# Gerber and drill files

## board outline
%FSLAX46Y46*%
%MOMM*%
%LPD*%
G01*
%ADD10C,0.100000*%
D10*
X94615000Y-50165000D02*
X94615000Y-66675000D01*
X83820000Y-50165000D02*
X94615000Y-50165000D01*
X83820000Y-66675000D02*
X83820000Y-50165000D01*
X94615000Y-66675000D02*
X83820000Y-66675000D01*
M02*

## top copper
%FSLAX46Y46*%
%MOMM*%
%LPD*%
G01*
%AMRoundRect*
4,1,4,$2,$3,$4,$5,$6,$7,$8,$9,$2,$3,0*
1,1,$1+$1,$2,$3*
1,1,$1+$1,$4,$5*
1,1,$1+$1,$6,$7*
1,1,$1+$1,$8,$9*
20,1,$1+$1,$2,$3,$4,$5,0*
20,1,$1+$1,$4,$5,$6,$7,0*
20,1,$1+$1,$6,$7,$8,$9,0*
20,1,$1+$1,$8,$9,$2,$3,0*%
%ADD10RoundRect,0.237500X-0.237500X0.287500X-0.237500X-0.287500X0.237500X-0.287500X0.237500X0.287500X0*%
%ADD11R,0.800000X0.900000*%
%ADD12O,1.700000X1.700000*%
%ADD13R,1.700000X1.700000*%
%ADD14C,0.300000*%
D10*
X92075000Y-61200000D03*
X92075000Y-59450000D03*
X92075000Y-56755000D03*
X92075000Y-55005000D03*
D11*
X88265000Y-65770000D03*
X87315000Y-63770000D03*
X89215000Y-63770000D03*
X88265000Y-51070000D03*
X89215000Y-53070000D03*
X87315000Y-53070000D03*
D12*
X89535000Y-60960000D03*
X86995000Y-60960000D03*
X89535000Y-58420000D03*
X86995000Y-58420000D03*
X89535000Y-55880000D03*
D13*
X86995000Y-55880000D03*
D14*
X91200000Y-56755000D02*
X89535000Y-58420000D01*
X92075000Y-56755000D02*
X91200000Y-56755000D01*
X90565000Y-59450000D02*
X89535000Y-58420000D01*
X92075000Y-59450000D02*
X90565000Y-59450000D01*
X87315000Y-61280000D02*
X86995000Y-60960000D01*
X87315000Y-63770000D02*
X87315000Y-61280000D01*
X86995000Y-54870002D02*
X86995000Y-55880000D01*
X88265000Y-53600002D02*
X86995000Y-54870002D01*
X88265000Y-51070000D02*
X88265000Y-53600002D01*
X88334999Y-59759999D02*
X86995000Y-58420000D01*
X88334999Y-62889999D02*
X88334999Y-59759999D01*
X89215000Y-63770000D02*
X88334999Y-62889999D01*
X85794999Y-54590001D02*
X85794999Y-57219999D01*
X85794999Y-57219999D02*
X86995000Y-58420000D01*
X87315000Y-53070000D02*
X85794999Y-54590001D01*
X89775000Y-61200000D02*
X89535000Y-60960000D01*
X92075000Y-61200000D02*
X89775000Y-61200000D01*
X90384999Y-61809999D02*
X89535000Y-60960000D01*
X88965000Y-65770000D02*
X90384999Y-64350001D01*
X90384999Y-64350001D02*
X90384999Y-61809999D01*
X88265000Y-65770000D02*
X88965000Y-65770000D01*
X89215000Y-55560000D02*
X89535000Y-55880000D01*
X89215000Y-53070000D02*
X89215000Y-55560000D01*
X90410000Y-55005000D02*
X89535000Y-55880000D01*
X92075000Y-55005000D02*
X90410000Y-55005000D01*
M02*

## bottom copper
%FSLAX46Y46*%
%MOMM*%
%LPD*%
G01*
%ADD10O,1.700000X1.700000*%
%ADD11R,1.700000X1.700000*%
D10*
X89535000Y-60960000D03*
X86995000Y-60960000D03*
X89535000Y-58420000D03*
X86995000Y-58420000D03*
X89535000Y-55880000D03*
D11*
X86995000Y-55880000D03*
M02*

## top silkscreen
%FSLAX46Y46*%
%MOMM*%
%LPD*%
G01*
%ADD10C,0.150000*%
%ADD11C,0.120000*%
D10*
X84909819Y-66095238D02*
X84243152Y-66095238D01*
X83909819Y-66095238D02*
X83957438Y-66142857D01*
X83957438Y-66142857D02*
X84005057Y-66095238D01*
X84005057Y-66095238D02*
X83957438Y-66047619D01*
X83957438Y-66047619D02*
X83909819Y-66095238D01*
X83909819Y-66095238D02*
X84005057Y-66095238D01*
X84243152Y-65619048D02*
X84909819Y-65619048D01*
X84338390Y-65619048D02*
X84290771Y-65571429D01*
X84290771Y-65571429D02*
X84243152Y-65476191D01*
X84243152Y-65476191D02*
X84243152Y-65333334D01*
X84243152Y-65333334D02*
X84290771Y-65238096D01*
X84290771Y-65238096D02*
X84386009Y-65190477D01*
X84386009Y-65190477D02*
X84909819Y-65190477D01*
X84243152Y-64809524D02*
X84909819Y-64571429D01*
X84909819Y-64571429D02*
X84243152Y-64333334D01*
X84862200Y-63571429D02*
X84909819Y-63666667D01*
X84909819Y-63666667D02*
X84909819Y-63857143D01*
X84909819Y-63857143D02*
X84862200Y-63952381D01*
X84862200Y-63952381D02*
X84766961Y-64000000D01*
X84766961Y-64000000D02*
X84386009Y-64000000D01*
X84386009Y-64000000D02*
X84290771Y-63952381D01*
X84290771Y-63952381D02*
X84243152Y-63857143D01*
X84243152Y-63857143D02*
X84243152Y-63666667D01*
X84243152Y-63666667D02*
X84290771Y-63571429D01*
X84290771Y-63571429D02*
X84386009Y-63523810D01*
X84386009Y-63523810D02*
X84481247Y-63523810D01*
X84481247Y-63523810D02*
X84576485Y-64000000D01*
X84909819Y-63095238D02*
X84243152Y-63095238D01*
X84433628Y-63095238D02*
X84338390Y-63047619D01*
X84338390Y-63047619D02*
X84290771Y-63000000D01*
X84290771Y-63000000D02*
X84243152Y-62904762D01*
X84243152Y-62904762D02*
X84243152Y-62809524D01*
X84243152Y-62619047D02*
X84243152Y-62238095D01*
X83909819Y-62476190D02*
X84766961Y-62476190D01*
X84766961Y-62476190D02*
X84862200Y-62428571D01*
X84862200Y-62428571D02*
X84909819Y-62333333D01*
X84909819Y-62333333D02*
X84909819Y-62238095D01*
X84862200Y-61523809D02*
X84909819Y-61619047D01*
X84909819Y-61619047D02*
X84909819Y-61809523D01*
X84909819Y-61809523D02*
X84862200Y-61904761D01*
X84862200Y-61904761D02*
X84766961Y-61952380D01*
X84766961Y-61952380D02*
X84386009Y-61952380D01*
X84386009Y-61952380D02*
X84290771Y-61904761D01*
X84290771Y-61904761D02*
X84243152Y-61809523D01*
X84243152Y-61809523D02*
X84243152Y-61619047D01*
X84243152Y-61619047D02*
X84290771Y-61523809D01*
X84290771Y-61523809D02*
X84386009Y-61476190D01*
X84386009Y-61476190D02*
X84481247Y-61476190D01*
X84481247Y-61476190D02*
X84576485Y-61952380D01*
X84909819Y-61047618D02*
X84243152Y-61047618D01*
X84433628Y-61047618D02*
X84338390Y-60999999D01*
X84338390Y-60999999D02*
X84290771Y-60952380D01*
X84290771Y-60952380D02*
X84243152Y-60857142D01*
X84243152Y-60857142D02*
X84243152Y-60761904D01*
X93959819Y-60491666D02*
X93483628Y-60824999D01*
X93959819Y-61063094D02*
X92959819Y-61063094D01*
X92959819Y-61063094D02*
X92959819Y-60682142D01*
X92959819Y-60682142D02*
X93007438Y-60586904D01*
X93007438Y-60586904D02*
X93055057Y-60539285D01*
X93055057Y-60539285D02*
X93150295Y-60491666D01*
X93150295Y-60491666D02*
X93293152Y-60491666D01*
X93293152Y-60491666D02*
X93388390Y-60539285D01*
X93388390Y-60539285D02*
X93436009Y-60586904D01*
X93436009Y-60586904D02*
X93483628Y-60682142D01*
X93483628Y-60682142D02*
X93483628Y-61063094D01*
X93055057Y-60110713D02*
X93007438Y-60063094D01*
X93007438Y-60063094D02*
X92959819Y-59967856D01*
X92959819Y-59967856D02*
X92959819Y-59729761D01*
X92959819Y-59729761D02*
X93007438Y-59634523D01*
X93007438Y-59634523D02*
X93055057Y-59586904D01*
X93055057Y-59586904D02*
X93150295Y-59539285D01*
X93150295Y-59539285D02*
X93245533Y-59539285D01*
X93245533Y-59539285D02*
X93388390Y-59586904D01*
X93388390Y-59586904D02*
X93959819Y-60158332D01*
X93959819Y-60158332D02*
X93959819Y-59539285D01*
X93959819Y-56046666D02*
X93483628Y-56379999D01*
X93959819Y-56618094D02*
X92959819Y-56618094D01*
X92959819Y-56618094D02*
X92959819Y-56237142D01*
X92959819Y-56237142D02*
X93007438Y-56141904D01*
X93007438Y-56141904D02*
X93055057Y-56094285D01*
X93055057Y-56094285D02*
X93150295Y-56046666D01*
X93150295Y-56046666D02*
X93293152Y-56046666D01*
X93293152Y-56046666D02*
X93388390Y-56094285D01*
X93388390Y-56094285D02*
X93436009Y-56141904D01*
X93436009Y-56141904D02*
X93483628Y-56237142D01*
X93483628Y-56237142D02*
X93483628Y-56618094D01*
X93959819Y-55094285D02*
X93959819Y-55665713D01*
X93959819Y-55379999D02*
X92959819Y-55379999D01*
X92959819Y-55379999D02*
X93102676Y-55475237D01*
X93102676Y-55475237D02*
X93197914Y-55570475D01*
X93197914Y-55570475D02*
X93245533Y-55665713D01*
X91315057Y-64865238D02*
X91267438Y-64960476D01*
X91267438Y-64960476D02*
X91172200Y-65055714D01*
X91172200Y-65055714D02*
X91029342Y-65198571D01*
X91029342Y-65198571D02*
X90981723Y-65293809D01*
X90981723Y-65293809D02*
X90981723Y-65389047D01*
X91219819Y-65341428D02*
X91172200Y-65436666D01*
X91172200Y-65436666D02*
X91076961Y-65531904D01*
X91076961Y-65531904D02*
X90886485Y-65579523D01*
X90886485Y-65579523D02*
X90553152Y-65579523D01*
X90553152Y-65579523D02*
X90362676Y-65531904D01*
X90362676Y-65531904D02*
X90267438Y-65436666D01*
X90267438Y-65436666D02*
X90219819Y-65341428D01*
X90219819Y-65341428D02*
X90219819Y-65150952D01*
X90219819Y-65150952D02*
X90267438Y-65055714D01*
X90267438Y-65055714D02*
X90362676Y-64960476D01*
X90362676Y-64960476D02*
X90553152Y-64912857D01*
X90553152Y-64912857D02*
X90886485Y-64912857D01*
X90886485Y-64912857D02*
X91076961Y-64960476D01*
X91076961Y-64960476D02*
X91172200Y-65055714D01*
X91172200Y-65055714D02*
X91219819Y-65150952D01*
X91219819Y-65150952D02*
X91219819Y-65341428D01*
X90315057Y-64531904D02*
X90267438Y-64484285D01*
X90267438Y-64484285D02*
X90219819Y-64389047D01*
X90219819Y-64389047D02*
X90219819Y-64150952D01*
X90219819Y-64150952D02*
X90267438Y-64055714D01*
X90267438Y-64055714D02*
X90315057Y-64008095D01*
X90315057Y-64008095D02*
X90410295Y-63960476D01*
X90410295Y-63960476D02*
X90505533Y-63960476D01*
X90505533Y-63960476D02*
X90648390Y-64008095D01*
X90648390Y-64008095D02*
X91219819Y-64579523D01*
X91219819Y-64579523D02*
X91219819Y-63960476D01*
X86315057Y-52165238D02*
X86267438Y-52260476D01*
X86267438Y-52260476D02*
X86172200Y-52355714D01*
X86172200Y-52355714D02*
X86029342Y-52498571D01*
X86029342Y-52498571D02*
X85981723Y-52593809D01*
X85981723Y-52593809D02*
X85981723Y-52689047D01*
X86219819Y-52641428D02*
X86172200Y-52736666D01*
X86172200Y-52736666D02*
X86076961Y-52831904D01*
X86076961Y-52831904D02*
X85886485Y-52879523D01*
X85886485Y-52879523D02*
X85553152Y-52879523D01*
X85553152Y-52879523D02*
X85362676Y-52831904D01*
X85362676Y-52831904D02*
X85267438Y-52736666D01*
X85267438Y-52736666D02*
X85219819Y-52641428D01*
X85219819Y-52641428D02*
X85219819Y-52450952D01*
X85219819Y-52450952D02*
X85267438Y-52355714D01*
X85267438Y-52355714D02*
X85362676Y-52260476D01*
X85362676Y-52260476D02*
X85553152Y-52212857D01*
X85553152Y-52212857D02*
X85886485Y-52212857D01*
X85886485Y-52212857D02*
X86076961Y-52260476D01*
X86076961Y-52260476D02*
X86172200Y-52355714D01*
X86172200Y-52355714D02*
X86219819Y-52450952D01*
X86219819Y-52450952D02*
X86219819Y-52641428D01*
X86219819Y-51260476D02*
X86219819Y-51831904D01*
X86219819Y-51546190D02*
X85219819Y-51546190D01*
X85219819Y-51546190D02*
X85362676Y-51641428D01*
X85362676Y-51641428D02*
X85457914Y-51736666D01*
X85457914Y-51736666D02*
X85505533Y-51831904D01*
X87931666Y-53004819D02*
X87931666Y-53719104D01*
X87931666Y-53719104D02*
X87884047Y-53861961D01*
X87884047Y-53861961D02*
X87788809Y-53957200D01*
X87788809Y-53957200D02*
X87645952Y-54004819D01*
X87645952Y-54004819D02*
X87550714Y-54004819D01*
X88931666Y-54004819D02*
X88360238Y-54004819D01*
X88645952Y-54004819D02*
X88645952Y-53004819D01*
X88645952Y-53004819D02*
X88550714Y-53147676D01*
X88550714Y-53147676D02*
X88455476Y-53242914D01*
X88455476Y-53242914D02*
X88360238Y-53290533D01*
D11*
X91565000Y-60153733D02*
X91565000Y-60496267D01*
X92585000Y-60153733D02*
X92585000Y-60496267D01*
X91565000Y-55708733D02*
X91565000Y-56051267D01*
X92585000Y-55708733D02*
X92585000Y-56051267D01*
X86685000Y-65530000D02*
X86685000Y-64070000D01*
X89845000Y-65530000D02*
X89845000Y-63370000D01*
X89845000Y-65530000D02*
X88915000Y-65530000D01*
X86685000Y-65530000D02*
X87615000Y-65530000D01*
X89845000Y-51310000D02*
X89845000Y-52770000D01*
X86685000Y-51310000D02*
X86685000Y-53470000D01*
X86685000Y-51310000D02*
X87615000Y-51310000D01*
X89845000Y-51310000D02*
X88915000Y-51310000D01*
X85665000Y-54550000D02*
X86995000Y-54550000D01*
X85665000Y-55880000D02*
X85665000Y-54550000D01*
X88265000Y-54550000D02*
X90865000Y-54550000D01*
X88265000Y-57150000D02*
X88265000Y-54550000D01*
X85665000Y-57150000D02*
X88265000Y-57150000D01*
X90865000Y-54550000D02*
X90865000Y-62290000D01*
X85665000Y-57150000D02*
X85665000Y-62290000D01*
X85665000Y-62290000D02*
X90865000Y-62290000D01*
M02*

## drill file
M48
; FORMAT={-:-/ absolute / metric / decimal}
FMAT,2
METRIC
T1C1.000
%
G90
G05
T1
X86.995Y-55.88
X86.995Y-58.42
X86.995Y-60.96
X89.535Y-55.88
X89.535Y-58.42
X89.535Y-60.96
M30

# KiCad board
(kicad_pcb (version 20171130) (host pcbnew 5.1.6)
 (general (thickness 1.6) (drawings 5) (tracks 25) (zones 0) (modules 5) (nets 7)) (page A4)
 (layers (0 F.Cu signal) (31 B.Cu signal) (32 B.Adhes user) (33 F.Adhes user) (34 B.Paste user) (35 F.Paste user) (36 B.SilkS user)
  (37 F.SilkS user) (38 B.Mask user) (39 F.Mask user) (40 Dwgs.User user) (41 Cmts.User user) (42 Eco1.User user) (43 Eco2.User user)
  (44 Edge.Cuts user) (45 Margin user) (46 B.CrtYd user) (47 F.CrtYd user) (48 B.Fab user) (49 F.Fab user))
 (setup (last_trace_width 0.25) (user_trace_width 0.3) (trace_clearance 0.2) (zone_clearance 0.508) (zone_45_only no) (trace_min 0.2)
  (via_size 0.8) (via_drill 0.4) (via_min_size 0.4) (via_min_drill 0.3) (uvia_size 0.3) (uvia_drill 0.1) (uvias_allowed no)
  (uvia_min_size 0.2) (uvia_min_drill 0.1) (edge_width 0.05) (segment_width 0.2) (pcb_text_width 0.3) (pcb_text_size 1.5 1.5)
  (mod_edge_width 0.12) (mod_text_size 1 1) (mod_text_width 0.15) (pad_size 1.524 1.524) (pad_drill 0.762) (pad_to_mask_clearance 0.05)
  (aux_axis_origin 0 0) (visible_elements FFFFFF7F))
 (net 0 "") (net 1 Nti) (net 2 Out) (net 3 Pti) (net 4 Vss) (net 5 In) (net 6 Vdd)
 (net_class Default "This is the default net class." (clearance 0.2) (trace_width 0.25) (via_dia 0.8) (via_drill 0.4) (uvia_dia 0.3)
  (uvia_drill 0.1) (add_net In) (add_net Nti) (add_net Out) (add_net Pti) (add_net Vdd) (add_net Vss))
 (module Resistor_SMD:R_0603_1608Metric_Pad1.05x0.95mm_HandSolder (layer F.Cu) (at 92.075 60.325 270)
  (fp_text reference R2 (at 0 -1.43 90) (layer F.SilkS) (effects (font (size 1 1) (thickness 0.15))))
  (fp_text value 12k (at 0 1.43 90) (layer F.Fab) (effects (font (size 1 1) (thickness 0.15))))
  (fp_line (start -0.171267 0.51) (end 0.171267 0.51) (layer F.SilkS) (width 0.12))
  (fp_line (start -0.171267 -0.51) (end 0.171267 -0.51) (layer F.SilkS) (width 0.12))
  (pad 2 smd roundrect (at 0.875 0 270) (size 1.05 0.95) (layers F.Cu F.Paste F.Mask) (roundrect_rratio 0.25) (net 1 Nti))
  (pad 1 smd roundrect (at -0.875 0 270) (size 1.05 0.95) (layers F.Cu F.Paste F.Mask) (roundrect_rratio 0.25) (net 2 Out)))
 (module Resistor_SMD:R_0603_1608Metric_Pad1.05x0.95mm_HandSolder (layer F.Cu) (at 92.075 55.88 270)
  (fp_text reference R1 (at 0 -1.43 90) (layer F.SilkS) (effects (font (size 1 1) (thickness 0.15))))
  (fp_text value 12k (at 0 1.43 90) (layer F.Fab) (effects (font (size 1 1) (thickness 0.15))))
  (fp_line (start -0.171267 0.51) (end 0.171267 0.51) (layer F.SilkS) (width 0.12))
  (fp_line (start -0.171267 -0.51) (end 0.171267 -0.51) (layer F.SilkS) (width 0.12))
  (pad 2 smd roundrect (at 0.875 0 270) (size 1.05 0.95) (layers F.Cu F.Paste F.Mask) (roundrect_rratio 0.25) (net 2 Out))
  (pad 1 smd roundrect (at -0.875 0 270) (size 1.05 0.95) (layers F.Cu F.Paste F.Mask) (roundrect_rratio 0.25) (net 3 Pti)))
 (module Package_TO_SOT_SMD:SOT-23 (layer F.Cu) (at 88.265 64.77 270)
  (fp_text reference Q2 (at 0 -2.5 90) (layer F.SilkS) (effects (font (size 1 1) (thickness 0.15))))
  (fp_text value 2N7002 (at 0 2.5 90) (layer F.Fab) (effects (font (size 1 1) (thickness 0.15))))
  (fp_line (start 0.76 1.58) (end -0.7 1.58) (layer F.SilkS) (width 0.12))
  (fp_line (start 0.76 -1.58) (end -1.4 -1.58) (layer F.SilkS) (width 0.12))
  (fp_line (start 0.76 -1.58) (end 0.76 -0.65) (layer F.SilkS) (width 0.12))
  (fp_line (start 0.76 1.58) (end 0.76 0.65) (layer F.SilkS) (width 0.12))
  (pad 3 smd rect (at 1 0 270) (size 0.9 0.8) (layers F.Cu F.Paste F.Mask) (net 1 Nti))
  (pad 2 smd rect (at -1 0.95 270) (size 0.9 0.8) (layers F.Cu F.Paste F.Mask) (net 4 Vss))
  (pad 1 smd rect (at -1 -0.95 270) (size 0.9 0.8) (layers F.Cu F.Paste F.Mask) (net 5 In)))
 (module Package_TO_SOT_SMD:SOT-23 (layer F.Cu) (at 88.265 52.07 90)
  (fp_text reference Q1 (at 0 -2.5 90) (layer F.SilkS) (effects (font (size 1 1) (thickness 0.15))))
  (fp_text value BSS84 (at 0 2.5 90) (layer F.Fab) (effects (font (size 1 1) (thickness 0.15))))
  (fp_line (start 0.76 1.58) (end -0.7 1.58) (layer F.SilkS) (width 0.12))
  (fp_line (start 0.76 -1.58) (end -1.4 -1.58) (layer F.SilkS) (width 0.12))
  (fp_line (start 0.76 -1.58) (end 0.76 -0.65) (layer F.SilkS) (width 0.12))
  (fp_line (start 0.76 1.58) (end 0.76 0.65) (layer F.SilkS) (width 0.12))
  (pad 3 smd rect (at 1 0 90) (size 0.9 0.8) (layers F.Cu F.Paste F.Mask) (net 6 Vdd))
  (pad 2 smd rect (at -1 0.95 90) (size 0.9 0.8) (layers F.Cu F.Paste F.Mask) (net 3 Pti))
  (pad 1 smd rect (at -1 -0.95 90) (size 0.9 0.8) (layers F.Cu F.Paste F.Mask) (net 5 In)))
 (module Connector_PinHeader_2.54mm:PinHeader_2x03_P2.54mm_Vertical (layer F.Cu) (at 86.995 55.88)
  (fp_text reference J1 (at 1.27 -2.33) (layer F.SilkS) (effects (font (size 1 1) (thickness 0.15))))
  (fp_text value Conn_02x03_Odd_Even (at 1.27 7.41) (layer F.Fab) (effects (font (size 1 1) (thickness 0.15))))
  (fp_line (start -1.33 -1.33) (end 0 -1.33) (layer F.SilkS) (width 0.12))
  (fp_line (start -1.33 0) (end -1.33 -1.33) (layer F.SilkS) (width 0.12))
  (fp_line (start 1.27 -1.33) (end 3.87 -1.33) (layer F.SilkS) (width 0.12))
  (fp_line (start 1.27 1.27) (end 1.27 -1.33) (layer F.SilkS) (width 0.12))
  (fp_line (start -1.33 1.27) (end 1.27 1.27) (layer F.SilkS) (width 0.12))
  (fp_line (start 3.87 -1.33) (end 3.87 6.41) (layer F.SilkS) (width 0.12))
  (fp_line (start -1.33 1.27) (end -1.33 6.41) (layer F.SilkS) (width 0.12))
  (fp_line (start -1.33 6.41) (end 3.87 6.41) (layer F.SilkS) (width 0.12))
  (pad 6 thru_hole oval (at 2.54 5.08) (size 1.7 1.7) (drill 1) (layers *.Cu *.Mask) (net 1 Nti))
  (pad 5 thru_hole oval (at 0 5.08) (size 1.7 1.7) (drill 1) (layers *.Cu *.Mask) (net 4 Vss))
  (pad 4 thru_hole oval (at 2.54 2.54) (size 1.7 1.7) (drill 1) (layers *.Cu *.Mask) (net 2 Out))
  (pad 3 thru_hole oval (at 0 2.54) (size 1.7 1.7) (drill 1) (layers *.Cu *.Mask) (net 5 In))
  (pad 2 thru_hole oval (at 2.54 0) (size 1.7 1.7) (drill 1) (layers *.Cu *.Mask) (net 3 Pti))
  (pad 1 thru_hole rect (at 0 0) (size 1.7 1.7) (drill 1) (layers *.Cu *.Mask) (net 6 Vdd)))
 (gr_line (start 94.615 50.165) (end 94.615 66.675) (layer Edge.Cuts) (width 0.1))
 (gr_line (start 83.82 50.165) (end 94.615 50.165) (layer Edge.Cuts) (width 0.1))
 (gr_line (start 83.82 66.675) (end 83.82 50.165) (layer Edge.Cuts) (width 0.1))
 (gr_line (start 94.615 66.675) (end 83.82 66.675) (layer Edge.Cuts) (width 0.1))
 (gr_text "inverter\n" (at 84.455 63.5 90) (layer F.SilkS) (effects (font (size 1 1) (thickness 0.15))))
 (segment (start 91.2 56.755) (end 89.535 58.42) (width 0.3) (layer F.Cu) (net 2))
 (segment (start 92.075 56.755) (end 91.2 56.755) (width 0.3) (layer F.Cu) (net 2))
 (segment (start 90.565 59.45) (end 89.535 58.42) (width 0.3) (layer F.Cu) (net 2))
 (segment (start 92.075 59.45) (end 90.565 59.45) (width 0.3) (layer F.Cu) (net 2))
 (segment (start 87.315 61.28) (end 86.995 60.96) (width 0.3) (layer F.Cu) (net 4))
 (segment (start 87.315 63.77) (end 87.315 61.28) (width 0.3) (layer F.Cu) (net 4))
 (segment (start 86.995 54.870002) (end 86.995 55.88) (width 0.3) (layer F.Cu) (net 6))
 (segment (start 88.265 53.600002) (end 86.995 54.870002) (width 0.3) (layer F.Cu) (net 6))
 (segment (start 88.265 51.07) (end 88.265 53.600002) (width 0.3) (layer F.Cu) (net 6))
 (segment (start 88.334999 59.759999) (end 86.995 58.42) (width 0.3) (layer F.Cu) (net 5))
 (segment (start 88.334999 62.889999) (end 88.334999 59.759999) (width 0.3) (layer F.Cu) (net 5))
 (segment (start 89.215 63.77) (end 88.334999 62.889999) (width 0.3) (layer F.Cu) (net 5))
 (segment (start 85.794999 54.590001) (end 85.794999 57.219999) (width 0.3) (layer F.Cu) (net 5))
 (segment (start 85.794999 57.219999) (end 86.995 58.42) (width 0.3) (layer F.Cu) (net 5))
 (segment (start 87.315 53.07) (end 85.794999 54.590001) (width 0.3) (layer F.Cu) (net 5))
 (segment (start 89.775 61.2) (end 89.535 60.96) (width 0.3) (layer F.Cu) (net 1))
 (segment (start 92.075 61.2) (end 89.775 61.2) (width 0.3) (layer F.Cu) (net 1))
 (segment (start 90.384999 61.809999) (end 89.535 60.96) (width 0.3) (layer F.Cu) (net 1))
 (segment (start 88.965 65.77) (end 90.384999 64.350001) (width 0.3) (layer F.Cu) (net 1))
 (segment (start 90.384999 64.350001) (end 90.384999 61.809999) (width 0.3) (layer F.Cu) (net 1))
 (segment (start 88.265 65.77) (end 88.965 65.77) (width 0.3) (layer F.Cu) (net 1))
 (segment (start 89.215 55.56) (end 89.535 55.88) (width 0.3) (layer F.Cu) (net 3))
 (segment (start 89.215 53.07) (end 89.215 55.56) (width 0.3) (layer F.Cu) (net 3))
 (segment (start 90.41 55.005) (end 89.535 55.88) (width 0.3) (layer F.Cu) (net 3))
 (segment (start 92.075 55.005) (end 90.41 55.005) (width 0.3) (layer F.Cu) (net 3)))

